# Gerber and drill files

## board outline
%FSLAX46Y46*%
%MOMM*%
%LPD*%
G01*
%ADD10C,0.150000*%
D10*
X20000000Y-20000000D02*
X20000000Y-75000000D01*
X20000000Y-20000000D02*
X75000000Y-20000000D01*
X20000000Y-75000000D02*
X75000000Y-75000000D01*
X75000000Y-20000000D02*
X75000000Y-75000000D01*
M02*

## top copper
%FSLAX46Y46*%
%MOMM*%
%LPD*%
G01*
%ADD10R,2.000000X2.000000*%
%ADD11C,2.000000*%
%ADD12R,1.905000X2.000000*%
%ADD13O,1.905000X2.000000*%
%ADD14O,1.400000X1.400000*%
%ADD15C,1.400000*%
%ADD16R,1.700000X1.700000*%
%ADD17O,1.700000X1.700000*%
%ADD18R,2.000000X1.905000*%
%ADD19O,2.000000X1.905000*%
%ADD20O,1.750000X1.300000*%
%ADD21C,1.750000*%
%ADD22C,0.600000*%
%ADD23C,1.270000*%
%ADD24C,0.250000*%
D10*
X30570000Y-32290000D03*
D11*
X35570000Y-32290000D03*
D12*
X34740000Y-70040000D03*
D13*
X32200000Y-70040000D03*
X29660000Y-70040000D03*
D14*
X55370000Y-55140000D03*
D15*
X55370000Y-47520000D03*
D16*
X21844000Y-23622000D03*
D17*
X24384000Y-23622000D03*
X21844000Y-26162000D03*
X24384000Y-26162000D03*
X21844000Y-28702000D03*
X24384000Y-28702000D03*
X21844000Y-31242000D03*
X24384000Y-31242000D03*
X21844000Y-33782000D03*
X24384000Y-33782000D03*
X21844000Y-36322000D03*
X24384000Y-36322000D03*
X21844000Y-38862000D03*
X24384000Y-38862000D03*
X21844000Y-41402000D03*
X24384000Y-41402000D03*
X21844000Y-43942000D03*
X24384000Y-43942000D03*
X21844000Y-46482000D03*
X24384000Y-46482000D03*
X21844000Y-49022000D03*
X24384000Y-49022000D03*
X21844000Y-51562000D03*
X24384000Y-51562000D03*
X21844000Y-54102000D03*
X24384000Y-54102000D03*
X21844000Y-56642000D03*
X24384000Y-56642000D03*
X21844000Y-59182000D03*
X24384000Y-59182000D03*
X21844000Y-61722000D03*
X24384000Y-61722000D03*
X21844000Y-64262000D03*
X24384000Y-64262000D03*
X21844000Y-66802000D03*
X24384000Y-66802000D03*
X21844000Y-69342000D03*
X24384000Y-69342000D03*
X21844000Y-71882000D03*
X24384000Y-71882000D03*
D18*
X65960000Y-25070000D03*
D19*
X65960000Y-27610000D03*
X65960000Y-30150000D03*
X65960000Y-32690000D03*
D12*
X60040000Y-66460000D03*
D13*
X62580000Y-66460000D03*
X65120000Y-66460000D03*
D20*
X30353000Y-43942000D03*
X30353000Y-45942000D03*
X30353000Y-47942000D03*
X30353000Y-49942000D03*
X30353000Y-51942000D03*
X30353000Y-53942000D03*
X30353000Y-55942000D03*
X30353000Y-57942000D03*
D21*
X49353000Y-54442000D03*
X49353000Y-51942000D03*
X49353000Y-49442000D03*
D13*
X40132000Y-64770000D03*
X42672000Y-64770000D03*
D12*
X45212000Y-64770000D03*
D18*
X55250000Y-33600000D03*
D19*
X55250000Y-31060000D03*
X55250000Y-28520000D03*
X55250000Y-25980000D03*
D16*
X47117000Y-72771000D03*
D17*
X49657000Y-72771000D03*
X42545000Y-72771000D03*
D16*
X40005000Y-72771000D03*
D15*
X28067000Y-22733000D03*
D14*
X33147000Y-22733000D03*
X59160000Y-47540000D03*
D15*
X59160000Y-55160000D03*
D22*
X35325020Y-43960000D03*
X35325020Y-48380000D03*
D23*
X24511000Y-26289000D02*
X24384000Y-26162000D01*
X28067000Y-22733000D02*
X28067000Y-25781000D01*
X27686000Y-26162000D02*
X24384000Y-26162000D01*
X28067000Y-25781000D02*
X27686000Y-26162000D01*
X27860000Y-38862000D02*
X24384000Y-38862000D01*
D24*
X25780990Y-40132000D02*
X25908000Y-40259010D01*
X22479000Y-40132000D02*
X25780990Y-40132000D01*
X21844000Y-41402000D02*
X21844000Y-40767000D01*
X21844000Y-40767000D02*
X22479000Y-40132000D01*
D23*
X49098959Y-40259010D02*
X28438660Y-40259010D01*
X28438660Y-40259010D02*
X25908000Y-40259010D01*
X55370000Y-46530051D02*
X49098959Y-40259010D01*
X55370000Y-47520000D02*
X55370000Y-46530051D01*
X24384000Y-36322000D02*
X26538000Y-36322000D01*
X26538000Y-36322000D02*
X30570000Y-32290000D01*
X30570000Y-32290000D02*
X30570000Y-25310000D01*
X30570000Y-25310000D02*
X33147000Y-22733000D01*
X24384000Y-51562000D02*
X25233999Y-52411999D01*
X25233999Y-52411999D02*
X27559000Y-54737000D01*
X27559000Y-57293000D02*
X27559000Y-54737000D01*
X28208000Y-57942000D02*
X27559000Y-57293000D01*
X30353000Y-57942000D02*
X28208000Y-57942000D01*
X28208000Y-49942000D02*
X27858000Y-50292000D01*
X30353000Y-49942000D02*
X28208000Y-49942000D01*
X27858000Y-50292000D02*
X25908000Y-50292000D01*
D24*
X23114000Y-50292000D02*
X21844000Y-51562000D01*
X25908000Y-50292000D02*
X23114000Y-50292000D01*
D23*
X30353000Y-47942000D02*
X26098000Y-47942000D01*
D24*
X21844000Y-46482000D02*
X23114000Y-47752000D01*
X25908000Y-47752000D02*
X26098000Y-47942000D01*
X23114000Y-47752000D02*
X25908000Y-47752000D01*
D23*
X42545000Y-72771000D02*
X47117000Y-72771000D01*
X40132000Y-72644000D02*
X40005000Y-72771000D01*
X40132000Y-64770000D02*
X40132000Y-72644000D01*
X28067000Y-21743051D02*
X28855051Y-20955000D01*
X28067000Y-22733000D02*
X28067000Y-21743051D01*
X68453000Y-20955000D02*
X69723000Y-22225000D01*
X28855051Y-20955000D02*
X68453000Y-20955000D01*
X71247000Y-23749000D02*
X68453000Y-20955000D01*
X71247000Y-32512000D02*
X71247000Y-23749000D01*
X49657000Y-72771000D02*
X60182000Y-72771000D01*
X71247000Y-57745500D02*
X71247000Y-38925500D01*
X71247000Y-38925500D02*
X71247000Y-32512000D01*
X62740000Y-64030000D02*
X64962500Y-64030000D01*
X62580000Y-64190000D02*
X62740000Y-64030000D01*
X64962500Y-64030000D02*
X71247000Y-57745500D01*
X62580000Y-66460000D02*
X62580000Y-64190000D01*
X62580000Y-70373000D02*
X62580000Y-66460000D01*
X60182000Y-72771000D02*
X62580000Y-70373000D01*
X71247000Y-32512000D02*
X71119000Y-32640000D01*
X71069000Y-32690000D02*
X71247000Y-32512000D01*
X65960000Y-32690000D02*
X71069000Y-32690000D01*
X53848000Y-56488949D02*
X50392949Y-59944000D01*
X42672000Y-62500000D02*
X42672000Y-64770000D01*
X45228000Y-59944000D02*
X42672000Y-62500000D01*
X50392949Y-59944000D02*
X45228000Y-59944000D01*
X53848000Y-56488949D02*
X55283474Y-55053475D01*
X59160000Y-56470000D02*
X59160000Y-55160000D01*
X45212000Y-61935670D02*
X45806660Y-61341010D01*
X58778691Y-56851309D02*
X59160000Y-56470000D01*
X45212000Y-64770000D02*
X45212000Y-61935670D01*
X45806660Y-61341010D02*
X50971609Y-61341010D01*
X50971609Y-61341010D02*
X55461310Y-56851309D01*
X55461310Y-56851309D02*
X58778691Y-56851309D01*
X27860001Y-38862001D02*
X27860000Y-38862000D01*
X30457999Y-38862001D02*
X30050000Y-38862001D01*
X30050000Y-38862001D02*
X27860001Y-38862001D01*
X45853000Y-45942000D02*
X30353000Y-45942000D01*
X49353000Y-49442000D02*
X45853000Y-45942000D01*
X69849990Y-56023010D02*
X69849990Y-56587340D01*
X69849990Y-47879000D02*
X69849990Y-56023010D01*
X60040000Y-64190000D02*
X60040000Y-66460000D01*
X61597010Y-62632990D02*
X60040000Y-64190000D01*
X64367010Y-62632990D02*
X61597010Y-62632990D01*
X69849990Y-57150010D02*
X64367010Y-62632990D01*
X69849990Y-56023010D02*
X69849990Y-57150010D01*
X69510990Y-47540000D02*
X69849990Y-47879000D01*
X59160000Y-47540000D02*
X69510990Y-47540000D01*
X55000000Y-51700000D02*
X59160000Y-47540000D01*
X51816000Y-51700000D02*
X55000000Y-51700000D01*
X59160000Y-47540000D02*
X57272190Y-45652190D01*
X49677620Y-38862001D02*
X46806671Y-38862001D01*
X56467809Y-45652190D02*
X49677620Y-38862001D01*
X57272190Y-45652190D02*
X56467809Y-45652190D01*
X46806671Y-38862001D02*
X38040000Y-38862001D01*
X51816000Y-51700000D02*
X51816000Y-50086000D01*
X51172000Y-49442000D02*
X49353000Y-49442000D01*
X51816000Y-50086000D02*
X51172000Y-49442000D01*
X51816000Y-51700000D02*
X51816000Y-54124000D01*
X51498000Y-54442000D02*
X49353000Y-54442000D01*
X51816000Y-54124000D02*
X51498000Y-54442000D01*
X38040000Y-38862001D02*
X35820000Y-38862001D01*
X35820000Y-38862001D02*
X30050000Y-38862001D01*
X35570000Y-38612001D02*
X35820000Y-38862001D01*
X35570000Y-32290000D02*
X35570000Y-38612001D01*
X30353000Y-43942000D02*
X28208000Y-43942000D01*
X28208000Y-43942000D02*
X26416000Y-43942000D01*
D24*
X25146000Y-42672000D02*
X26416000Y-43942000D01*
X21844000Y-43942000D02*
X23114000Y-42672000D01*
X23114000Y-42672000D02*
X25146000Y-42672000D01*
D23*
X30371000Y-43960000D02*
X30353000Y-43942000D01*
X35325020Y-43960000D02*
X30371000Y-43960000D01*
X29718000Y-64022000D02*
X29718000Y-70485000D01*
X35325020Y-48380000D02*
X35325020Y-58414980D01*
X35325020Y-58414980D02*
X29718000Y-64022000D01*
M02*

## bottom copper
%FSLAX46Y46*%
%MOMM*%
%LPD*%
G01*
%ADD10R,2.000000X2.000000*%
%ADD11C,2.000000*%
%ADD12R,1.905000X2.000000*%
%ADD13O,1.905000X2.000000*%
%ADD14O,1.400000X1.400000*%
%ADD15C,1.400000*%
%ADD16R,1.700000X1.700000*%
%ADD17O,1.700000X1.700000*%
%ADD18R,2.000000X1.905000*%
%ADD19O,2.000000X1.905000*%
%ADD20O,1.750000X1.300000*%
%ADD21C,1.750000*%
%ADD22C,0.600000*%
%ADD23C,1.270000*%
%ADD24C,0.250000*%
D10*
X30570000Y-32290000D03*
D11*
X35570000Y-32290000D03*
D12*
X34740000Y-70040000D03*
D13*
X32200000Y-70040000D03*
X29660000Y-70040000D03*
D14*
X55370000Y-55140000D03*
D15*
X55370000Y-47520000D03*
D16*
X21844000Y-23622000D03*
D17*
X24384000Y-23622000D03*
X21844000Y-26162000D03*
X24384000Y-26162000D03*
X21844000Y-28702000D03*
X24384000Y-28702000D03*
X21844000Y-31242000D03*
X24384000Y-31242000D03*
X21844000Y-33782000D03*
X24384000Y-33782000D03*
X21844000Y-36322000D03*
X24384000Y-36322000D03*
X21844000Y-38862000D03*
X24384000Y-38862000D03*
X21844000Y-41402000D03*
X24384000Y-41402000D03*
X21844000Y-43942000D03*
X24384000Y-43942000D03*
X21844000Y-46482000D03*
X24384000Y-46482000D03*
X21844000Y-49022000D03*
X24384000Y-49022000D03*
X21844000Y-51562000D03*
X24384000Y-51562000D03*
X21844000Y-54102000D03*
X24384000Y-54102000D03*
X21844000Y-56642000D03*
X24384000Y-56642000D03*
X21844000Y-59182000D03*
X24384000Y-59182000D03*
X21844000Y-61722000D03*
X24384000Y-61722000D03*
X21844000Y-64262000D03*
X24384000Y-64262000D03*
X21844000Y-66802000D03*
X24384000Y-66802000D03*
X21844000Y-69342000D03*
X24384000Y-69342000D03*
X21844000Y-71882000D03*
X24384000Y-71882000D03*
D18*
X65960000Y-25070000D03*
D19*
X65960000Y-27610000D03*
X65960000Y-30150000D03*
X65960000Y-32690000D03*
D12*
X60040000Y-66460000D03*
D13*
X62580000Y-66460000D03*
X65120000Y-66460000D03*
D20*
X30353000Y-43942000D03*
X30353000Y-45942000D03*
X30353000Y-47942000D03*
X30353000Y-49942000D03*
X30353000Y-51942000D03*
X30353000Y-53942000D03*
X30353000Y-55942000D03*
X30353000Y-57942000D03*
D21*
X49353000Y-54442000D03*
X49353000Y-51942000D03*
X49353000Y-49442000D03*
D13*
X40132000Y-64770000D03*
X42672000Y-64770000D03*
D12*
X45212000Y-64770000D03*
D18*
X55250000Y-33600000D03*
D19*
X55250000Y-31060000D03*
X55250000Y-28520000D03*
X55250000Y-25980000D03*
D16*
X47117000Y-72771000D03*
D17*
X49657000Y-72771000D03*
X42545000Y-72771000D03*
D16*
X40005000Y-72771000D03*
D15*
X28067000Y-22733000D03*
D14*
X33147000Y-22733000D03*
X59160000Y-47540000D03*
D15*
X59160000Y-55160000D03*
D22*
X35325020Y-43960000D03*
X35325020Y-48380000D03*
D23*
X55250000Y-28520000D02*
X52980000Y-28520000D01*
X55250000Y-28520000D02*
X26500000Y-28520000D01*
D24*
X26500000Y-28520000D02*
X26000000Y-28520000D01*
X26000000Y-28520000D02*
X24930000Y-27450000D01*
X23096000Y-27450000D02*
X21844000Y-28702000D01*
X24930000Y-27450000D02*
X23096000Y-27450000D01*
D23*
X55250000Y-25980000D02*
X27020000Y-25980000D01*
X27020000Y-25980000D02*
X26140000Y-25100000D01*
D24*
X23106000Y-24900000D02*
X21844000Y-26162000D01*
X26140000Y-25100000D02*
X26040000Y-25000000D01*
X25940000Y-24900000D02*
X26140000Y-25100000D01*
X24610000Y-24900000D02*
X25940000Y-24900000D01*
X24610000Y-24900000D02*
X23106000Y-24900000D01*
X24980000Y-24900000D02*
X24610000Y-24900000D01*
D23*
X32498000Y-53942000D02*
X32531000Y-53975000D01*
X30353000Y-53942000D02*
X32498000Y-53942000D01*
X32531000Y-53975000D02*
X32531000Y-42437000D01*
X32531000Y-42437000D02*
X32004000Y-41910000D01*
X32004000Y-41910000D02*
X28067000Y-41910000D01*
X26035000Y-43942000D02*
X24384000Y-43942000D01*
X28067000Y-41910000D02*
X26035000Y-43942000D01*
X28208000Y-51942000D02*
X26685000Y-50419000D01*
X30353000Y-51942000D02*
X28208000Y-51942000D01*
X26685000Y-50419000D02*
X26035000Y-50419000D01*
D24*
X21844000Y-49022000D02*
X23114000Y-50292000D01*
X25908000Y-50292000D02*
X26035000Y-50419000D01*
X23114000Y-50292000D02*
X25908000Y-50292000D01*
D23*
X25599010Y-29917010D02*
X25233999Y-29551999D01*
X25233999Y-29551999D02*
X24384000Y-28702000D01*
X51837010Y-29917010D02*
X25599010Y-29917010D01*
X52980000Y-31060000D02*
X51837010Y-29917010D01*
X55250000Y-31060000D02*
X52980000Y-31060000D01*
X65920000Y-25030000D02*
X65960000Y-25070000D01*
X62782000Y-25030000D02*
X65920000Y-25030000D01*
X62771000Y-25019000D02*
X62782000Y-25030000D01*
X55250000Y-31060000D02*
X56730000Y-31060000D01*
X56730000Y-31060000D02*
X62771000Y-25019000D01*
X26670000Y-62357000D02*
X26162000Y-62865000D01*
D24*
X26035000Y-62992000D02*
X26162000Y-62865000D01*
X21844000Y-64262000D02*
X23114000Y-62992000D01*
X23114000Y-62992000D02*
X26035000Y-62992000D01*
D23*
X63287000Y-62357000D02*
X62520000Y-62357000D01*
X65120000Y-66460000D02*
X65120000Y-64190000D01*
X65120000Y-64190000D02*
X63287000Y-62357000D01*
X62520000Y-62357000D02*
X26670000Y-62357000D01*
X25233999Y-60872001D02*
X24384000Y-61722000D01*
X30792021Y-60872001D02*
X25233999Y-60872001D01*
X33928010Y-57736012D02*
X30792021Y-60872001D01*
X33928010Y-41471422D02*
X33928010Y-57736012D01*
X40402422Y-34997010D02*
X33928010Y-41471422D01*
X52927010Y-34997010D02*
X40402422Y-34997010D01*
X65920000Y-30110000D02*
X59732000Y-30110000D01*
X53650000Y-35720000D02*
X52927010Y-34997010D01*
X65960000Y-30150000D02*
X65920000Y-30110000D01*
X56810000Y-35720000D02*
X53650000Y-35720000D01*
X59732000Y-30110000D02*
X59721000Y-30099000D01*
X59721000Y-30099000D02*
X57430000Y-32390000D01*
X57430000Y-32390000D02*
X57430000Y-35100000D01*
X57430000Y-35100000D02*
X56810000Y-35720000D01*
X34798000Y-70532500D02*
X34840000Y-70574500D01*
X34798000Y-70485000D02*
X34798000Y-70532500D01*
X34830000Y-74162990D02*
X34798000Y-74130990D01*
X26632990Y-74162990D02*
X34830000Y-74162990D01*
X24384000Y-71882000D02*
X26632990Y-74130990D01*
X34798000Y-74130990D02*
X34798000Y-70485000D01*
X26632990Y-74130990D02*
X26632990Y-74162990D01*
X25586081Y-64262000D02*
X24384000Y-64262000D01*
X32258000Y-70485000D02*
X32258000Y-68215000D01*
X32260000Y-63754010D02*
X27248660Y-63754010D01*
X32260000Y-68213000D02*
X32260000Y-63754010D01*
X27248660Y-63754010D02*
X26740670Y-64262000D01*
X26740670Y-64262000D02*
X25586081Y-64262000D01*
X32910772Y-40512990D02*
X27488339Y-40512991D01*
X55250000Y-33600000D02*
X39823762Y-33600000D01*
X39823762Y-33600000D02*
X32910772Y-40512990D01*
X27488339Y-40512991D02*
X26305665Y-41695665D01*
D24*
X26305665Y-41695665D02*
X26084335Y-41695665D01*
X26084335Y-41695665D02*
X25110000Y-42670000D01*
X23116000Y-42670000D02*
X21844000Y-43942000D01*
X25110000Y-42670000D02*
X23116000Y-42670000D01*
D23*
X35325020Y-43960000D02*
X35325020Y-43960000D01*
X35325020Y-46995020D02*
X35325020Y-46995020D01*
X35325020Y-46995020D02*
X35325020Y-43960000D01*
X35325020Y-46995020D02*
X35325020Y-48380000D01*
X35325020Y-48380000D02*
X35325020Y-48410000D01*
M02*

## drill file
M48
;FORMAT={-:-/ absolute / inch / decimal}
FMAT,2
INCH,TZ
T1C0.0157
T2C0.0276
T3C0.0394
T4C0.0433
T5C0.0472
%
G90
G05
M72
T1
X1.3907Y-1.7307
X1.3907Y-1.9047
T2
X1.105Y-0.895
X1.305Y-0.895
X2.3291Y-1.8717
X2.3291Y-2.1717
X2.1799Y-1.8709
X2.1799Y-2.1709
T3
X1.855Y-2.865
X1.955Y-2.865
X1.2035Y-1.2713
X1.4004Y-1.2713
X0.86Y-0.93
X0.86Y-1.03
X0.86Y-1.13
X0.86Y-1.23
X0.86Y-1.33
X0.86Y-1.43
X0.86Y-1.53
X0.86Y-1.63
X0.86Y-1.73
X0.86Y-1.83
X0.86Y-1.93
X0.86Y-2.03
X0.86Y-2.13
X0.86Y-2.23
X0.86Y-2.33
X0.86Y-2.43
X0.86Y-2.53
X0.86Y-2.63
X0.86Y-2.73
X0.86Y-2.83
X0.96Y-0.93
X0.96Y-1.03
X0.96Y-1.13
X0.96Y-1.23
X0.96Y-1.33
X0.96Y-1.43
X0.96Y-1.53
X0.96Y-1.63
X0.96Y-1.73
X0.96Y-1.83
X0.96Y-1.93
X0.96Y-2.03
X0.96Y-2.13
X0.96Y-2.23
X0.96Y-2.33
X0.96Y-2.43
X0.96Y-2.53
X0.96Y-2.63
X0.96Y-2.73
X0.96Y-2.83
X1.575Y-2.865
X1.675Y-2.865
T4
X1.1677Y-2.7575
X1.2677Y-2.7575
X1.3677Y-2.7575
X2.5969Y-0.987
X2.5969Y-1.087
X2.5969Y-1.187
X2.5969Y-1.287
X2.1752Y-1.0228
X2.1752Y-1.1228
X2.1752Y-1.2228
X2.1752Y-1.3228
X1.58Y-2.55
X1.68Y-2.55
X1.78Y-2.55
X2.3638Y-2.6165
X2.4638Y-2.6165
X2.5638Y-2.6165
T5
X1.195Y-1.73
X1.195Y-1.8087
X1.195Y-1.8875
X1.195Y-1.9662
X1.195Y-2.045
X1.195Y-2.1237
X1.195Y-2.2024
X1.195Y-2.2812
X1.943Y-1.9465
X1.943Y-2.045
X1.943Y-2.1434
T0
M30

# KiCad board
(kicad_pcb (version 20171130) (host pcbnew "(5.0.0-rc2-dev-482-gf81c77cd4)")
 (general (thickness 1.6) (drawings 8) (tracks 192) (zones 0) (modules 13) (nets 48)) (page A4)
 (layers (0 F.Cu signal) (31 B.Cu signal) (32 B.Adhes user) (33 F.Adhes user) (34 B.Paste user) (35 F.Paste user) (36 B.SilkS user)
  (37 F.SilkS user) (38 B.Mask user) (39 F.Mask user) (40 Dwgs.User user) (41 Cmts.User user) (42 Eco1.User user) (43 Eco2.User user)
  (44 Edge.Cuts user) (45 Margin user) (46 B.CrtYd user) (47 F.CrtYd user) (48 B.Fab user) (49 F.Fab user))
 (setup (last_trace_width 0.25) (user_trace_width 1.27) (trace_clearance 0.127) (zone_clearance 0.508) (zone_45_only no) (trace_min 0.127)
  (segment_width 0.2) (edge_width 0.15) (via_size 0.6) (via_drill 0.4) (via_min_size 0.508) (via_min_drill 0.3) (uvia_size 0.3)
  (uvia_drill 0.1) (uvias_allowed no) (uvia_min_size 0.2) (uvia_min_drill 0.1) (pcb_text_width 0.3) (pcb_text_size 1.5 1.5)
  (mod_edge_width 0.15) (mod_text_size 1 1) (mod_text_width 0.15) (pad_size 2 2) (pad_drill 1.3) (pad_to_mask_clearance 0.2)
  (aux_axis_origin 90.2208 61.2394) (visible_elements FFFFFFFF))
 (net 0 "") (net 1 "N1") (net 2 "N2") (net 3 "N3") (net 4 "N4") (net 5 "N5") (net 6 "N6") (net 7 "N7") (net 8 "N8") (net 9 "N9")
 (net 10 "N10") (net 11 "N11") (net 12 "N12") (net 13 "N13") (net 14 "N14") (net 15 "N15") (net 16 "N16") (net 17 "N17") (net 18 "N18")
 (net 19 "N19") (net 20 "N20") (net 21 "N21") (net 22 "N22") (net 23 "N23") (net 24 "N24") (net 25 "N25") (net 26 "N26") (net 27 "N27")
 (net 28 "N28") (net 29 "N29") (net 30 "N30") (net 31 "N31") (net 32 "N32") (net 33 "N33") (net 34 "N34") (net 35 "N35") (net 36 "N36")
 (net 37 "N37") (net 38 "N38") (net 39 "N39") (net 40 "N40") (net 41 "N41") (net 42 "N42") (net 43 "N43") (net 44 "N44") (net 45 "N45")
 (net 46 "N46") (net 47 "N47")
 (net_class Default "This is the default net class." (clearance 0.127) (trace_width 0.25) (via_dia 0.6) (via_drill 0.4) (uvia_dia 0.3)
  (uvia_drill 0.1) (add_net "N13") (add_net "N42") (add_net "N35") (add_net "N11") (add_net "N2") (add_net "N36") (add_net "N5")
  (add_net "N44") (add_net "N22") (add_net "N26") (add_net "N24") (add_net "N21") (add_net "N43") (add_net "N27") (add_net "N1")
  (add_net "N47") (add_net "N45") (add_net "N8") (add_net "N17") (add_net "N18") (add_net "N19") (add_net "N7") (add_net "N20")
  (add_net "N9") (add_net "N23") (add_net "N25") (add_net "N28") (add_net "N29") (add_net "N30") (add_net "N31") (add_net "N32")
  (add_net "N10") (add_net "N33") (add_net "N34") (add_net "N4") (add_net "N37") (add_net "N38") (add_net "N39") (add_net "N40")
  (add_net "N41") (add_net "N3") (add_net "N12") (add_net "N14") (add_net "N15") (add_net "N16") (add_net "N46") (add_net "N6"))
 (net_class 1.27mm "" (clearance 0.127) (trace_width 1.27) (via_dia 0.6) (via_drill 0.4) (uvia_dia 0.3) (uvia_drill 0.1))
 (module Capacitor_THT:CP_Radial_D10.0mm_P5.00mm (layer F.Cu) (at 30.57 32.29)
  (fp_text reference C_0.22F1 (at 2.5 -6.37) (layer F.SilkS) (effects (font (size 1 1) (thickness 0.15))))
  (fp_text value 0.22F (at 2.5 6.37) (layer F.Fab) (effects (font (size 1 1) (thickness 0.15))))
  (pad 1 thru_hole rect (at 0 0) (size 2 2) (drill 1) (layers *.Cu *.Mask) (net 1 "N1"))
  (pad 2 thru_hole circle (at 5 0) (size 2 2) (drill 1) (layers *.Cu *.Mask) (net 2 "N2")))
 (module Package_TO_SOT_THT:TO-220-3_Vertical (layer F.Cu) (at 34.74 70.04 180)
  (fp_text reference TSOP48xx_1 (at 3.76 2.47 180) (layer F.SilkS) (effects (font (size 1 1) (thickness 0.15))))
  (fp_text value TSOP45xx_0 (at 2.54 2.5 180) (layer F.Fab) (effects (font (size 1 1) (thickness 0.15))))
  (pad 1 thru_hole rect (at 0 0 180) (size 1.905 2) (drill 1.1) (layers *.Cu *.Mask) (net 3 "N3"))
  (pad 2 thru_hole oval (at 2.54 0 180) (size 1.905 2) (drill 1.1) (layers *.Cu *.Mask) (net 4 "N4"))
  (pad 3 thru_hole oval (at 5.08 0 180) (size 1.905 2) (drill 1.1) (layers *.Cu *.Mask) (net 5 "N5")))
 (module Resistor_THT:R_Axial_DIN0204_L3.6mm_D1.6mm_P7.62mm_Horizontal (layer F.Cu) (at 55.37 47.52 270)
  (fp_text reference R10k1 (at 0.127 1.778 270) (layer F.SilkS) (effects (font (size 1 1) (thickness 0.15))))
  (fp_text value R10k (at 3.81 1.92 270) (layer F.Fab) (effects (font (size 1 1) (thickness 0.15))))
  (pad 2 thru_hole oval (at 7.62 0 270) (size 1.4 1.4) (drill 0.7) (layers *.Cu *.Mask) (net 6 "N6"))
  (pad 1 thru_hole circle (at 0 0 270) (size 1.4 1.4) (drill 0.7) (layers *.Cu *.Mask) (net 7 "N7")))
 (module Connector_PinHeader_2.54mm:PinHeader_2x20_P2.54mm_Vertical (layer F.Cu) (at 21.844 23.622)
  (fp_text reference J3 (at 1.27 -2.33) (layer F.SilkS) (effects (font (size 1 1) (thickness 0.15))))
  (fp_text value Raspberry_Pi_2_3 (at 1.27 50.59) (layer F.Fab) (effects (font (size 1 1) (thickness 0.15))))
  (pad 1 thru_hole rect (at 0 0) (size 1.7 1.7) (drill 1) (layers *.Cu *.Mask) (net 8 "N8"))
  (pad 2 thru_hole oval (at 2.54 0) (size 1.7 1.7) (drill 1) (layers *.Cu *.Mask) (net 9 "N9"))
  (pad 3 thru_hole oval (at 0 2.54) (size 1.7 1.7) (drill 1) (layers *.Cu *.Mask) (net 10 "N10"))
  (pad 4 thru_hole oval (at 2.54 2.54) (size 1.7 1.7) (drill 1) (layers *.Cu *.Mask) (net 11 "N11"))
  (pad 5 thru_hole oval (at 0 5.08) (size 1.7 1.7) (drill 1) (layers *.Cu *.Mask) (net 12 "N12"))
  (pad 6 thru_hole oval (at 2.54 5.08) (size 1.7 1.7) (drill 1) (layers *.Cu *.Mask) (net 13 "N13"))
  (pad 7 thru_hole oval (at 0 7.62) (size 1.7 1.7) (drill 1) (layers *.Cu *.Mask) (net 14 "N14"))
  (pad 8 thru_hole oval (at 2.54 7.62) (size 1.7 1.7) (drill 1) (layers *.Cu *.Mask) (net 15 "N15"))
  (pad 9 thru_hole oval (at 0 10.16) (size 1.7 1.7) (drill 1) (layers *.Cu *.Mask) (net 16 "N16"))
  (pad 10 thru_hole oval (at 2.54 10.16) (size 1.7 1.7) (drill 1) (layers *.Cu *.Mask) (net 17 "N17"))
  (pad 11 thru_hole oval (at 0 12.7) (size 1.7 1.7) (drill 1) (layers *.Cu *.Mask) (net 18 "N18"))
  (pad 12 thru_hole oval (at 2.54 12.7) (size 1.7 1.7) (drill 1) (layers *.Cu *.Mask) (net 1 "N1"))
  (pad 13 thru_hole oval (at 0 15.24) (size 1.7 1.7) (drill 1) (layers *.Cu *.Mask) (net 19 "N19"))
  (pad 14 thru_hole oval (at 2.54 15.24) (size 1.7 1.7) (drill 1) (layers *.Cu *.Mask) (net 2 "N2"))
  (pad 15 thru_hole oval (at 0 17.78) (size 1.7 1.7) (drill 1) (layers *.Cu *.Mask) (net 7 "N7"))
  (pad 16 thru_hole oval (at 2.54 17.78) (size 1.7 1.7) (drill 1) (layers *.Cu *.Mask) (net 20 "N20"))
  (pad 17 thru_hole oval (at 0 20.32) (size 1.7 1.7) (drill 1) (layers *.Cu *.Mask) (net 5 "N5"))
  (pad 18 thru_hole oval (at 2.54 20.32) (size 1.7 1.7) (drill 1) (layers *.Cu *.Mask) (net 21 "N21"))
  (pad 19 thru_hole oval (at 0 22.86) (size 1.7 1.7) (drill 1) (layers *.Cu *.Mask) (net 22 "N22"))
  (pad 20 thru_hole oval (at 2.54 22.86) (size 1.7 1.7) (drill 1) (layers *.Cu *.Mask) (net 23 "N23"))
  (pad 21 thru_hole oval (at 0 25.4) (size 1.7 1.7) (drill 1) (layers *.Cu *.Mask) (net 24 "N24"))
  (pad 22 thru_hole oval (at 2.54 25.4) (size 1.7 1.7) (drill 1) (layers *.Cu *.Mask) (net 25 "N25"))
  (pad 23 thru_hole oval (at 0 27.94) (size 1.7 1.7) (drill 1) (layers *.Cu *.Mask) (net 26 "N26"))
  (pad 24 thru_hole oval (at 2.54 27.94) (size 1.7 1.7) (drill 1) (layers *.Cu *.Mask) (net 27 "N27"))
  (pad 25 thru_hole oval (at 0 30.48) (size 1.7 1.7) (drill 1) (layers *.Cu *.Mask) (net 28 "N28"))
  (pad 26 thru_hole oval (at 2.54 30.48) (size 1.7 1.7) (drill 1) (layers *.Cu *.Mask) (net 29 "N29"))
  (pad 27 thru_hole oval (at 0 33.02) (size 1.7 1.7) (drill 1) (layers *.Cu *.Mask) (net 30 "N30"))
  (pad 28 thru_hole oval (at 2.54 33.02) (size 1.7 1.7) (drill 1) (layers *.Cu *.Mask) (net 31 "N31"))
  (pad 29 thru_hole oval (at 0 35.56) (size 1.7 1.7) (drill 1) (layers *.Cu *.Mask) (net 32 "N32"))
  (pad 30 thru_hole oval (at 2.54 35.56) (size 1.7 1.7) (drill 1) (layers *.Cu *.Mask) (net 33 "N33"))
  (pad 31 thru_hole oval (at 0 38.1) (size 1.7 1.7) (drill 1) (layers *.Cu *.Mask) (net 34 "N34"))
  (pad 32 thru_hole oval (at 2.54 38.1) (size 1.7 1.7) (drill 1) (layers *.Cu *.Mask) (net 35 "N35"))
  (pad 33 thru_hole oval (at 0 40.64) (size 1.7 1.7) (drill 1) (layers *.Cu *.Mask) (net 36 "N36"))
  (pad 34 thru_hole oval (at 2.54 40.64) (size 1.7 1.7) (drill 1) (layers *.Cu *.Mask) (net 4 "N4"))
  (pad 35 thru_hole oval (at 0 43.18) (size 1.7 1.7) (drill 1) (layers *.Cu *.Mask) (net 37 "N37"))
  (pad 36 thru_hole oval (at 2.54 43.18) (size 1.7 1.7) (drill 1) (layers *.Cu *.Mask) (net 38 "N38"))
  (pad 37 thru_hole oval (at 0 45.72) (size 1.7 1.7) (drill 1) (layers *.Cu *.Mask) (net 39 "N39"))
  (pad 38 thru_hole oval (at 2.54 45.72) (size 1.7 1.7) (drill 1) (layers *.Cu *.Mask) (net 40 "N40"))
  (pad 39 thru_hole oval (at 0 48.26) (size 1.7 1.7) (drill 1) (layers *.Cu *.Mask) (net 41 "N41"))
  (pad 40 thru_hole oval (at 2.54 48.26) (size 1.7 1.7) (drill 1) (layers *.Cu *.Mask) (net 3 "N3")))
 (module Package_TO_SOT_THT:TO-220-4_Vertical (layer F.Cu) (at 65.96 25.07 270)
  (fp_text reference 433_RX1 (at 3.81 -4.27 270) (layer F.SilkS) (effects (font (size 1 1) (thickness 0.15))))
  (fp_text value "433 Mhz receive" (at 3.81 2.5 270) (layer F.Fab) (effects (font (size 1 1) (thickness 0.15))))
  (pad 1 thru_hole rect (at 0 0 270) (size 1.905 2) (drill 1.1) (layers *.Cu *.Mask) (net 13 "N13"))
  (pad 2 thru_hole oval (at 2.54 0 270) (size 1.905 2) (drill 1.1) (layers *.Cu *.Mask) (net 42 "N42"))
  (pad 3 thru_hole oval (at 5.08 0 270) (size 1.905 2) (drill 1.1) (layers *.Cu *.Mask) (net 35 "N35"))
  (pad 4 thru_hole oval (at 7.62 0 270) (size 1.905 2) (drill 1.1) (layers *.Cu *.Mask) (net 11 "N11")))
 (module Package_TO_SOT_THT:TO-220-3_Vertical (layer F.Cu) (at 60.04 66.46)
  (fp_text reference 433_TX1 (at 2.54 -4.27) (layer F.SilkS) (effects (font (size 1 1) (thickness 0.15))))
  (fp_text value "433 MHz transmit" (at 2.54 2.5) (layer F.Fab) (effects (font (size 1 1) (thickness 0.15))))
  (pad 1 thru_hole rect (at 0 0) (size 1.905 2) (drill 1.1) (layers *.Cu *.Mask) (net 2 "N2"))
  (pad 2 thru_hole oval (at 2.54 0) (size 1.905 2) (drill 1.1) (layers *.Cu *.Mask) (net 11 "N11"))
  (pad 3 thru_hole oval (at 5.08 0) (size 1.905 2) (drill 1.1) (layers *.Cu *.Mask) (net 36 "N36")))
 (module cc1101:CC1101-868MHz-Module (layer F.Cu) (at 39.853 50.942)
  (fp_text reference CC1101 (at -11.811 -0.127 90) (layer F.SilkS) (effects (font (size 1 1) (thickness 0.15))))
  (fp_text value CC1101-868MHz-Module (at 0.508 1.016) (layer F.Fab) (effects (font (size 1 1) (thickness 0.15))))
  (pad 1 thru_hole oval (at -9.5 -7) (size 1.75 1.3) (drill 1.2) (layers *.Cu *.Mask) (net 5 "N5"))
  (pad 2 thru_hole oval (at -9.5 -5) (size 1.75 1.3) (drill 1.2) (layers *.Cu *.Mask) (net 2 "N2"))
  (pad 3 thru_hole oval (at -9.5 -3) (size 1.75 1.3) (drill 1.2) (layers *.Cu *.Mask) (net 22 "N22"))
  (pad 4 thru_hole oval (at -9.5 -1) (size 1.75 1.3) (drill 1.2) (layers *.Cu *.Mask) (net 26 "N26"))
  (pad 5 thru_hole oval (at -9.5 1) (size 1.75 1.3) (drill 1.2) (layers *.Cu *.Mask) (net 24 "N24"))
  (pad 6 thru_hole oval (at -9.5 3) (size 1.75 1.3) (drill 1.2) (layers *.Cu *.Mask) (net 21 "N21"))
  (pad 7 thru_hole oval (at -9.5 5) (size 1.75 1.3) (drill 1.2) (layers *.Cu *.Mask) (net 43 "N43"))
  (pad 8 thru_hole oval (at -9.5 7) (size 1.75 1.3) (drill 1.2) (layers *.Cu *.Mask) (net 27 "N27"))
  (pad 9 thru_hole circle (at 9.5 3.5) (size 1.75 1.75) (drill 1.2) (layers *.Cu *.Mask) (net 2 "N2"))
  (pad 10 thru_hole circle (at 9.5 1) (size 1.75 1.75) (drill 1.2) (layers *.Cu *.Mask) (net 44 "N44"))
  (pad 11 thru_hole circle (at 9.5 -1.5) (size 1.75 1.75) (drill 1.2) (layers *.Cu *.Mask) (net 2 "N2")))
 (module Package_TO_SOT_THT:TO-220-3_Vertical (layer F.Cu) (at 45.212 64.77 180)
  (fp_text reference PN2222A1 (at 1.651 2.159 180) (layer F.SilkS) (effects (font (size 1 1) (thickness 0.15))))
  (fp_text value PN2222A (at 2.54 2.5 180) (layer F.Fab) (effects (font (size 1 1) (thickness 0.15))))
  (pad 3 thru_hole oval (at 5.08 0 180) (size 1.905 2) (drill 1.1) (layers *.Cu *.Mask) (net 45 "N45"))
  (pad 2 thru_hole oval (at 2.54 0 180) (size 1.905 2) (drill 1.1) (layers *.Cu *.Mask) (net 6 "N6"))
  (pad 1 thru_hole rect (at 0 0 180) (size 1.905 2) (drill 1.1) (layers *.Cu *.Mask) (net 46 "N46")))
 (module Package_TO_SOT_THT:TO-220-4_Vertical (layer F.Cu) (at 55.25 33.6 90)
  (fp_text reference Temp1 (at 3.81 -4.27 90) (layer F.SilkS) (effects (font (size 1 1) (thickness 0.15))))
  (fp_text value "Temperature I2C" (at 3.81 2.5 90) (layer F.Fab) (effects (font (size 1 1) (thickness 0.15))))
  (pad 1 thru_hole rect (at 0 0 90) (size 1.905 2) (drill 1.1) (layers *.Cu *.Mask) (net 5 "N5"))
  (pad 2 thru_hole oval (at 2.54 0 90) (size 1.905 2) (drill 1.1) (layers *.Cu *.Mask) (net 13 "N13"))
  (pad 3 thru_hole oval (at 5.08 0 90) (size 1.905 2) (drill 1.1) (layers *.Cu *.Mask) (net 12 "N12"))
  (pad 4 thru_hole oval (at 7.62 0 90) (size 1.905 2) (drill 1.1) (layers *.Cu *.Mask) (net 10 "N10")))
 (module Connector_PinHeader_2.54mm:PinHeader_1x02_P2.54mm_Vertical (layer F.Cu) (at 47.117 72.771 90)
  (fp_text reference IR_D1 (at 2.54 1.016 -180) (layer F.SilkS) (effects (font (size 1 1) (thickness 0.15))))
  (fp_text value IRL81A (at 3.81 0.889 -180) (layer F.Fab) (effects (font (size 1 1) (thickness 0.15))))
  (pad 1 thru_hole rect (at 0 0 90) (size 1.7 1.7) (drill 1) (layers *.Cu *.Mask) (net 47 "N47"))
  (pad 2 thru_hole oval (at 0 2.54 90) (size 1.7 1.7) (drill 1) (layers *.Cu *.Mask) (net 11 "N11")))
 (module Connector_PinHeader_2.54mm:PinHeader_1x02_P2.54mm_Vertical (layer F.Cu) (at 40.005 72.771 90)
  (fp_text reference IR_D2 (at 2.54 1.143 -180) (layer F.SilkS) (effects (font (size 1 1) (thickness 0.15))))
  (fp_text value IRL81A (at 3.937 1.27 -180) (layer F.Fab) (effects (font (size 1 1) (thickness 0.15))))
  (pad 2 thru_hole oval (at 0 2.54 90) (size 1.7 1.7) (drill 1) (layers *.Cu *.Mask) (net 47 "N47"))
  (pad 1 thru_hole rect (at 0 0 90) (size 1.7 1.7) (drill 1) (layers *.Cu *.Mask) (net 45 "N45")))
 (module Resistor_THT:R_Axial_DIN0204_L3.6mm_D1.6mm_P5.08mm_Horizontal (layer F.Cu) (at 28.067 22.733)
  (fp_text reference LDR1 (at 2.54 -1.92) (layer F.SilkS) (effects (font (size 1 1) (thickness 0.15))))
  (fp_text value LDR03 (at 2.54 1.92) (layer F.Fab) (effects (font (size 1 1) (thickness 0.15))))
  (pad 1 thru_hole circle (at 0 0) (size 1.4 1.4) (drill 0.7) (layers *.Cu *.Mask) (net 11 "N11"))
  (pad 2 thru_hole oval (at 5.08 0) (size 1.4 1.4) (drill 0.7) (layers *.Cu *.Mask) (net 1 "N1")))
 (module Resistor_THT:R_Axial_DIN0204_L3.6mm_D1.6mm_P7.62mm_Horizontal (layer F.Cu) (at 59.16 55.16 90)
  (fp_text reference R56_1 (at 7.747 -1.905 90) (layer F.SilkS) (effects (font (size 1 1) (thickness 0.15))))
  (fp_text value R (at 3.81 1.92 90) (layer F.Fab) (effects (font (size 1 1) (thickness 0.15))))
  (pad 2 thru_hole oval (at 7.62 0 90) (size 1.4 1.4) (drill 0.7) (layers *.Cu *.Mask) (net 2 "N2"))
  (pad 1 thru_hole circle (at 0 0 90) (size 1.4 1.4) (drill 0.7) (layers *.Cu *.Mask) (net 46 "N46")))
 (gr_line (start 20 20) (end 20 75) (angle 90) (layer Edge.Cuts) (width 0.15))
 (gr_line (start 20 20) (end 75 20) (angle 90) (layer Edge.Cuts) (width 0.15))
 (gr_line (start 20 75) (end 75 75) (angle 90) (layer Edge.Cuts) (width 0.15))
 (gr_line (start 75 20) (end 75 75) (angle 90) (layer Edge.Cuts) (width 0.15))
 (segment (start 24.511 26.289) (end 24.384 26.162) (width 1.27) (layer F.Cu) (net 11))
 (segment (start 28.067 22.733) (end 28.067 25.781) (width 1.27) (layer F.Cu) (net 11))
 (segment (start 27.686 26.162) (end 24.384 26.162) (width 1.27) (layer F.Cu) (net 11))
 (segment (start 28.067 25.781) (end 27.686 26.162) (width 1.27) (layer F.Cu) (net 11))
 (segment (start 27.86 38.862) (end 24.384 38.862) (width 1.27) (layer F.Cu) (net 2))
 (segment (start 25.78099 40.132) (end 25.908 40.25901) (width 0.25) (layer F.Cu) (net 7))
 (segment (start 22.479 40.132) (end 25.78099 40.132) (width 0.25) (layer F.Cu) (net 7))
 (segment (start 21.844 41.402) (end 21.844 40.767) (width 0.25) (layer F.Cu) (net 7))
 (segment (start 21.844 40.767) (end 22.479 40.132) (width 0.25) (layer F.Cu) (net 7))
 (segment (start 49.098959 40.25901) (end 28.43866 40.25901) (width 1.27) (layer F.Cu) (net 7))
 (segment (start 28.43866 40.25901) (end 25.908 40.25901) (width 1.27) (layer F.Cu) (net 7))
 (segment (start 55.37 46.530051) (end 49.098959 40.25901) (width 1.27) (layer F.Cu) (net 7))
 (segment (start 55.37 47.52) (end 55.37 46.530051) (width 1.27) (layer F.Cu) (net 7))
 (segment (start 55.25 28.52) (end 52.98 28.52) (width 1.27) (layer B.Cu) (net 12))
 (segment (start 55.25 28.52) (end 26.5 28.52) (width 1.27) (layer B.Cu) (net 12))
 (segment (start 26.5 28.52) (end 26 28.52) (width 0.25) (layer B.Cu) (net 12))
 (segment (start 26 28.52) (end 24.93 27.45) (width 0.25) (layer B.Cu) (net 12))
 (segment (start 23.096 27.45) (end 21.844 28.702) (width 0.25) (layer B.Cu) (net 12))
 (segment (start 24.93 27.45) (end 23.096 27.45) (width 0.25) (layer B.Cu) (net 12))
 (segment (start 55.25 25.98) (end 27.02 25.98) (width 1.27) (layer B.Cu) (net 10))
 (segment (start 27.02 25.98) (end 26.14 25.1) (width 1.27) (layer B.Cu) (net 10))
 (segment (start 23.106 24.9) (end 21.844 26.162) (width 0.25) (layer B.Cu) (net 10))
 (segment (start 26.14 25.1) (end 26.04 25) (width 0.25) (layer B.Cu) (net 10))
 (segment (start 25.94 24.9) (end 26.14 25.1) (width 0.25) (layer B.Cu) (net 10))
 (segment (start 24.61 24.9) (end 25.94 24.9) (width 0.25) (layer B.Cu) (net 10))
 (segment (start 24.61 24.9) (end 23.106 24.9) (width 0.25) (layer B.Cu) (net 10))
 (segment (start 24.98 24.9) (end 24.61 24.9) (width 0.25) (layer B.Cu) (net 10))
 (segment (start 24.384 36.322) (end 26.538 36.322) (width 1.27) (layer F.Cu) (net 1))
 (segment (start 26.538 36.322) (end 30.57 32.29) (width 1.27) (layer F.Cu) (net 1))
 (segment (start 30.57 32.29) (end 30.57 25.31) (width 1.27) (layer F.Cu) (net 1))
 (segment (start 30.57 25.31) (end 33.147 22.733) (width 1.27) (layer F.Cu) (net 1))
 (segment (start 24.384 51.562) (end 25.233999 52.411999) (width 1.27) (layer F.Cu) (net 27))
 (segment (start 25.233999 52.411999) (end 27.559 54.737) (width 1.27) (layer F.Cu) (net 27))
 (segment (start 27.559 57.293) (end 27.559 54.737) (width 1.27) (layer F.Cu) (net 27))
 (segment (start 28.208 57.942) (end 27.559 57.293) (width 1.27) (layer F.Cu) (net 27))
 (segment (start 30.353 57.942) (end 28.208 57.942) (width 1.27) (layer F.Cu) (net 27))
 (segment (start 32.498 53.942) (end 32.531 53.975) (width 1.27) (layer B.Cu) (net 21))
 (segment (start 30.353 53.942) (end 32.498 53.942) (width 1.27) (layer B.Cu) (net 21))
 (segment (start 32.531 53.975) (end 32.531 42.437) (width 1.27) (layer B.Cu) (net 21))
 (segment (start 32.531 42.437) (end 32.004 41.91) (width 1.27) (layer B.Cu) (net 21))
 (segment (start 32.004 41.91) (end 28.067 41.91) (width 1.27) (layer B.Cu) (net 21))
 (segment (start 26.035 43.942) (end 24.384 43.942) (width 1.27) (layer B.Cu) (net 21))
 (segment (start 28.067 41.91) (end 26.035 43.942) (width 1.27) (layer B.Cu) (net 21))
 (segment (start 28.208 51.942) (end 26.685 50.419) (width 1.27) (layer B.Cu) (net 24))
 (segment (start 30.353 51.942) (end 28.208 51.942) (width 1.27) (layer B.Cu) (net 24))
 (segment (start 26.685 50.419) (end 26.035 50.419) (width 1.27) (layer B.Cu) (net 24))
 (segment (start 21.844 49.022) (end 23.114 50.292) (width 0.25) (layer B.Cu) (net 24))
 (segment (start 25.908 50.292) (end 26.035 50.419) (width 0.25) (layer B.Cu) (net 24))
 (segment (start 23.114 50.292) (end 25.908 50.292) (width 0.25) (layer B.Cu) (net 24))
 (segment (start 28.208 49.942) (end 27.858 50.292) (width 1.27) (layer F.Cu) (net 26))
 (segment (start 30.353 49.942) (end 28.208 49.942) (width 1.27) (layer F.Cu) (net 26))
 (segment (start 27.858 50.292) (end 25.908 50.292) (width 1.27) (layer F.Cu) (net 26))
 (segment (start 23.114 50.292) (end 21.844 51.562) (width 0.25) (layer F.Cu) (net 26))
 (segment (start 25.908 50.292) (end 23.114 50.292) (width 0.25) (layer F.Cu) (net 26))
 (segment (start 30.353 47.942) (end 26.098 47.942) (width 1.27) (layer F.Cu) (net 22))
 (segment (start 21.844 46.482) (end 23.114 47.752) (width 0.25) (layer F.Cu) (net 22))
 (segment (start 25.908 47.752) (end 26.098 47.942) (width 0.25) (layer F.Cu) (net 22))
 (segment (start 23.114 47.752) (end 25.908 47.752) (width 0.25) (layer F.Cu) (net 22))
 (segment (start 42.545 72.771) (end 47.117 72.771) (width 1.27) (layer F.Cu) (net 47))
 (segment (start 40.132 72.644) (end 40.005 72.771) (width 1.27) (layer F.Cu) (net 45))
 (segment (start 40.132 64.77) (end 40.132 72.644) (width 1.27) (layer F.Cu) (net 45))
 (segment (start 25.59901 29.91701) (end 25.233999 29.551999) (width 1.27) (layer B.Cu) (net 13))
 (segment (start 25.233999 29.551999) (end 24.384 28.702) (width 1.27) (layer B.Cu) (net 13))
 (segment (start 51.83701 29.91701) (end 25.59901 29.91701) (width 1.27) (layer B.Cu) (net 13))
 (segment (start 52.98 31.06) (end 51.83701 29.91701) (width 1.27) (layer B.Cu) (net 13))
 (segment (start 55.25 31.06) (end 52.98 31.06) (width 1.27) (layer B.Cu) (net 13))
 (segment (start 65.92 25.03) (end 65.96 25.07) (width 1.27) (layer B.Cu) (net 13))
 (segment (start 62.782 25.03) (end 65.92 25.03) (width 1.27) (layer B.Cu) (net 13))
 (segment (start 62.771 25.019) (end 62.782 25.03) (width 1.27) (layer B.Cu) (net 13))
 (segment (start 55.25 31.06) (end 56.73 31.06) (width 1.27) (layer B.Cu) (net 13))
 (segment (start 56.73 31.06) (end 62.771 25.019) (width 1.27) (layer B.Cu) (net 13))
 (segment (start 28.067 21.743051) (end 28.855051 20.955) (width 1.27) (layer F.Cu) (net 11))
 (segment (start 28.067 22.733) (end 28.067 21.743051) (width 1.27) (layer F.Cu) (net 11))
 (segment (start 68.453 20.955) (end 69.723 22.225) (width 1.27) (layer F.Cu) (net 11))
 (segment (start 28.855051 20.955) (end 68.453 20.955) (width 1.27) (layer F.Cu) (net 11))
 (segment (start 71.247 23.749) (end 68.453 20.955) (width 1.27) (layer F.Cu) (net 11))
 (segment (start 71.247 32.512) (end 71.247 23.749) (width 1.27) (layer F.Cu) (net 11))
 (segment (start 49.657 72.771) (end 60.182 72.771) (width 1.27) (layer F.Cu) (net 11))
 (segment (start 71.247 57.7455) (end 71.247 38.9255) (width 1.27) (layer F.Cu) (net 11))
 (segment (start 71.247 38.9255) (end 71.247 32.512) (width 1.27) (layer F.Cu) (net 11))
 (segment (start 62.74 64.03) (end 64.9625 64.03) (width 1.27) (layer F.Cu) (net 11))
 (segment (start 62.58 64.19) (end 62.74 64.03) (width 1.27) (layer F.Cu) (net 11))
 (segment (start 64.9625 64.03) (end 71.247 57.7455) (width 1.27) (layer F.Cu) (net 11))
 (segment (start 62.58 66.46) (end 62.58 64.19) (width 1.27) (layer F.Cu) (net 11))
 (segment (start 62.58 70.373) (end 62.58 66.46) (width 1.27) (layer F.Cu) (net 11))
 (segment (start 60.182 72.771) (end 62.58 70.373) (width 1.27) (layer F.Cu) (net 11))
 (segment (start 71.247 32.512) (end 71.119 32.64) (width 1.27) (layer F.Cu) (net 11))
 (segment (start 71.069 32.69) (end 71.247 32.512) (width 1.27) (layer F.Cu) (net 11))
 (segment (start 65.96 32.69) (end 71.069 32.69) (width 1.27) (layer F.Cu) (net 11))
 (segment (start 26.67 62.357) (end 26.162 62.865) (width 1.27) (layer B.Cu) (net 36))
 (segment (start 26.035 62.992) (end 26.162 62.865) (width 0.25) (layer B.Cu) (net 36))
 (segment (start 21.844 64.262) (end 23.114 62.992) (width 0.25) (layer B.Cu) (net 36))
 (segment (start 23.114 62.992) (end 26.035 62.992) (width 0.25) (layer B.Cu) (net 36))
 (segment (start 63.287 62.357) (end 62.52 62.357) (width 1.27) (layer B.Cu) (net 36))
 (segment (start 65.12 66.46) (end 65.12 64.19) (width 1.27) (layer B.Cu) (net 36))
 (segment (start 65.12 64.19) (end 63.287 62.357) (width 1.27) (layer B.Cu) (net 36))
 (segment (start 62.52 62.357) (end 26.67 62.357) (width 1.27) (layer B.Cu) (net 36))
 (segment (start 53.848 56.488949) (end 50.392949 59.944) (width 1.27) (layer F.Cu) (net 6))
 (segment (start 42.672 62.5) (end 42.672 64.77) (width 1.27) (layer F.Cu) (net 6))
 (segment (start 45.228 59.944) (end 42.672 62.5) (width 1.27) (layer F.Cu) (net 6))
 (segment (start 50.392949 59.944) (end 45.228 59.944) (width 1.27) (layer F.Cu) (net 6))
 (segment (start 53.848 56.488949) (end 55.283474 55.053475) (width 1.27) (layer F.Cu) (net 6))
 (segment (start 59.16 56.47) (end 59.16 55.16) (width 1.27) (layer F.Cu) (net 46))
 (segment (start 45.212 61.93567) (end 45.80666 61.34101) (width 1.27) (layer F.Cu) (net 46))
 (segment (start 58.778691 56.851309) (end 59.16 56.47) (width 1.27) (layer F.Cu) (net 46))
 (segment (start 45.212 64.77) (end 45.212 61.93567) (width 1.27) (layer F.Cu) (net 46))
 (segment (start 45.80666 61.34101) (end 50.971609 61.34101) (width 1.27) (layer F.Cu) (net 46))
 (segment (start 50.971609 61.34101) (end 55.46131 56.851309) (width 1.27) (layer F.Cu) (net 46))
 (segment (start 55.46131 56.851309) (end 58.778691 56.851309) (width 1.27) (layer F.Cu) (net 46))
 (segment (start 25.233999 60.872001) (end 24.384 61.722) (width 1.27) (layer B.Cu) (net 35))
 (segment (start 30.792021 60.872001) (end 25.233999 60.872001) (width 1.27) (layer B.Cu) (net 35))
 (segment (start 33.92801 57.736012) (end 30.792021 60.872001) (width 1.27) (layer B.Cu) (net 35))
 (segment (start 33.92801 41.471422) (end 33.92801 57.736012) (width 1.27) (layer B.Cu) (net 35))
 (segment (start 40.402422 34.99701) (end 33.92801 41.471422) (width 1.27) (layer B.Cu) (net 35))
 (segment (start 52.92701 34.99701) (end 40.402422 34.99701) (width 1.27) (layer B.Cu) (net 35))
 (segment (start 65.92 30.11) (end 59.732 30.11) (width 1.27) (layer B.Cu) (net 35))
 (segment (start 53.65 35.72) (end 52.92701 34.99701) (width 1.27) (layer B.Cu) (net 35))
 (segment (start 65.96 30.15) (end 65.92 30.11) (width 1.27) (layer B.Cu) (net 35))
 (segment (start 56.81 35.72) (end 53.65 35.72) (width 1.27) (layer B.Cu) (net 35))
 (segment (start 59.732 30.11) (end 59.721 30.099) (width 1.27) (layer B.Cu) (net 35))
 (segment (start 59.721 30.099) (end 57.43 32.39) (width 1.27) (layer B.Cu) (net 35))
 (segment (start 57.43 32.39) (end 57.43 35.1) (width 1.27) (layer B.Cu) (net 35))
 (segment (start 57.43 35.1) (end 56.81 35.72) (width 1.27) (layer B.Cu) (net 35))
 (segment (start 27.860001 38.862001) (end 27.86 38.862) (width 1.27) (layer F.Cu) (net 2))
 (segment (start 30.457999 38.862001) (end 30.05 38.862001) (width 1.27) (layer F.Cu) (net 2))
 (segment (start 30.05 38.862001) (end 27.860001 38.862001) (width 1.27) (layer F.Cu) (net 2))
 (segment (start 45.853 45.942) (end 30.353 45.942) (width 1.27) (layer F.Cu) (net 2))
 (segment (start 49.353 49.442) (end 45.853 45.942) (width 1.27) (layer F.Cu) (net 2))
 (segment (start 69.84999 56.02301) (end 69.84999 56.58734) (width 1.27) (layer F.Cu) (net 2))
 (segment (start 69.84999 47.879) (end 69.84999 56.02301) (width 1.27) (layer F.Cu) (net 2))
 (segment (start 60.04 64.19) (end 60.04 66.46) (width 1.27) (layer F.Cu) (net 2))
 (segment (start 61.59701 62.63299) (end 60.04 64.19) (width 1.27) (layer F.Cu) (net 2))
 (segment (start 64.36701 62.63299) (end 61.59701 62.63299) (width 1.27) (layer F.Cu) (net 2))
 (segment (start 69.84999 57.15001) (end 64.36701 62.63299) (width 1.27) (layer F.Cu) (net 2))
 (segment (start 69.84999 56.02301) (end 69.84999 57.15001) (width 1.27) (layer F.Cu) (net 2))
 (segment (start 69.51099 47.54) (end 69.84999 47.879) (width 1.27) (layer F.Cu) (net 2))
 (segment (start 59.16 47.54) (end 69.51099 47.54) (width 1.27) (layer F.Cu) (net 2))
 (segment (start 55 51.7) (end 59.16 47.54) (width 1.27) (layer F.Cu) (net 2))
 (segment (start 51.816 51.7) (end 55 51.7) (width 1.27) (layer F.Cu) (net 2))
 (segment (start 59.16 47.54) (end 57.27219 45.65219) (width 1.27) (layer F.Cu) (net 2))
 (segment (start 49.67762 38.862001) (end 46.806671 38.862001) (width 1.27) (layer F.Cu) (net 2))
 (segment (start 56.467809 45.65219) (end 49.67762 38.862001) (width 1.27) (layer F.Cu) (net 2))
 (segment (start 57.27219 45.65219) (end 56.467809 45.65219) (width 1.27) (layer F.Cu) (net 2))
 (segment (start 46.806671 38.862001) (end 38.04 38.862001) (width 1.27) (layer F.Cu) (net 2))
 (segment (start 51.816 51.7) (end 51.816 50.086) (width 1.27) (layer F.Cu) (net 2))
 (segment (start 51.172 49.442) (end 49.353 49.442) (width 1.27) (layer F.Cu) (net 2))
 (segment (start 51.816 50.086) (end 51.172 49.442) (width 1.27) (layer F.Cu) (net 2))
 (segment (start 51.816 51.7) (end 51.816 54.124) (width 1.27) (layer F.Cu) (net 2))
 (segment (start 51.498 54.442) (end 49.353 54.442) (width 1.27) (layer F.Cu) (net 2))
 (segment (start 51.816 54.124) (end 51.498 54.442) (width 1.27) (layer F.Cu) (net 2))
 (segment (start 38.04 38.862001) (end 35.82 38.862001) (width 1.27) (layer F.Cu) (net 2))
 (segment (start 35.82 38.862001) (end 30.05 38.862001) (width 1.27) (layer F.Cu) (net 2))
 (segment (start 35.57 38.612001) (end 35.82 38.862001) (width 1.27) (layer F.Cu) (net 2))
 (segment (start 35.57 32.29) (end 35.57 38.612001) (width 1.27) (layer F.Cu) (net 2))
 (segment (start 34.798 70.5325) (end 34.84 70.5745) (width 1.27) (layer B.Cu) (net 3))
 (segment (start 34.798 70.485) (end 34.798 70.5325) (width 1.27) (layer B.Cu) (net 3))
 (segment (start 34.83 74.16299) (end 34.798 74.13099) (width 1.27) (layer B.Cu) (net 3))
 (segment (start 26.63299 74.16299) (end 34.83 74.16299) (width 1.27) (layer B.Cu) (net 3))
 (segment (start 24.384 71.882) (end 26.63299 74.13099) (width 1.27) (layer B.Cu) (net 3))
 (segment (start 34.798 74.13099) (end 34.798 70.485) (width 1.27) (layer B.Cu) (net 3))
 (segment (start 26.63299 74.13099) (end 26.63299 74.16299) (width 1.27) (layer B.Cu) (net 3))
 (segment (start 25.586081 64.262) (end 24.384 64.262) (width 1.27) (layer B.Cu) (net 4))
 (segment (start 32.258 70.485) (end 32.258 68.215) (width 1.27) (layer B.Cu) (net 4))
 (segment (start 32.26 63.75401) (end 27.24866 63.75401) (width 1.27) (layer B.Cu) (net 4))
 (segment (start 32.26 68.213) (end 32.26 63.75401) (width 1.27) (layer B.Cu) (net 4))
 (segment (start 27.24866 63.75401) (end 26.74067 64.262) (width 1.27) (layer B.Cu) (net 4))
 (segment (start 26.74067 64.262) (end 25.586081 64.262) (width 1.27) (layer B.Cu) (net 4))
 (segment (start 30.353 43.942) (end 28.208 43.942) (width 1.27) (layer F.Cu) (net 5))
 (segment (start 28.208 43.942) (end 26.416 43.942) (width 1.27) (layer F.Cu) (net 5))
 (segment (start 25.146 42.672) (end 26.416 43.942) (width 0.25) (layer F.Cu) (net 5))
 (segment (start 21.844 43.942) (end 23.114 42.672) (width 0.25) (layer F.Cu) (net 5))
 (segment (start 23.114 42.672) (end 25.146 42.672) (width 0.25) (layer F.Cu) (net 5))
 (segment (start 32.910772 40.51299) (end 27.488339 40.512991) (width 1.27) (layer B.Cu) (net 5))
 (segment (start 55.25 33.6) (end 39.823762 33.6) (width 1.27) (layer B.Cu) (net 5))
 (segment (start 39.823762 33.6) (end 32.910772 40.51299) (width 1.27) (layer B.Cu) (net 5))
 (segment (start 27.488339 40.512991) (end 26.305665 41.695665) (width 1.27) (layer B.Cu) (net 5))
 (segment (start 26.305665 41.695665) (end 26.084335 41.695665) (width 0.25) (layer B.Cu) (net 5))
 (segment (start 26.084335 41.695665) (end 25.11 42.67) (width 0.25) (layer B.Cu) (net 5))
 (segment (start 23.116 42.67) (end 21.844 43.942) (width 0.25) (layer B.Cu) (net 5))
 (segment (start 25.11 42.67) (end 23.116 42.67) (width 0.25) (layer B.Cu) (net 5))
 (segment (start 35.32502 43.96) (end 35.32502 43.96) (width 1.27) (layer B.Cu) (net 5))
 (via (at 35.32502 43.96) (size 0.6) (drill 0.4) (layers F.Cu B.Cu) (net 5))
 (segment (start 30.371 43.96) (end 30.353 43.942) (width 1.27) (layer F.Cu) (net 5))
 (segment (start 35.32502 43.96) (end 30.371 43.96) (width 1.27) (layer F.Cu) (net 5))
 (segment (start 35.32502 46.99502) (end 35.32502 46.99502) (width 1.27) (layer B.Cu) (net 5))
 (segment (start 35.32502 46.99502) (end 35.32502 43.96) (width 1.27) (layer B.Cu) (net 5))
 (segment (start 35.32502 46.99502) (end 35.32502 48.38) (width 1.27) (layer B.Cu) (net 5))
 (segment (start 35.32502 48.38) (end 35.32502 48.41) (width 1.27) (layer B.Cu) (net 5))
 (via (at 35.32502 48.38) (size 0.6) (drill 0.4) (layers F.Cu B.Cu) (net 5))
 (segment (start 29.718 64.022) (end 29.718 70.485) (width 1.27) (layer F.Cu) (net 5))
 (segment (start 35.32502 48.38) (end 35.32502 58.41498) (width 1.27) (layer F.Cu) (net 5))
 (segment (start 35.32502 58.41498) (end 29.718 64.022) (width 1.27) (layer F.Cu) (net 5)))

